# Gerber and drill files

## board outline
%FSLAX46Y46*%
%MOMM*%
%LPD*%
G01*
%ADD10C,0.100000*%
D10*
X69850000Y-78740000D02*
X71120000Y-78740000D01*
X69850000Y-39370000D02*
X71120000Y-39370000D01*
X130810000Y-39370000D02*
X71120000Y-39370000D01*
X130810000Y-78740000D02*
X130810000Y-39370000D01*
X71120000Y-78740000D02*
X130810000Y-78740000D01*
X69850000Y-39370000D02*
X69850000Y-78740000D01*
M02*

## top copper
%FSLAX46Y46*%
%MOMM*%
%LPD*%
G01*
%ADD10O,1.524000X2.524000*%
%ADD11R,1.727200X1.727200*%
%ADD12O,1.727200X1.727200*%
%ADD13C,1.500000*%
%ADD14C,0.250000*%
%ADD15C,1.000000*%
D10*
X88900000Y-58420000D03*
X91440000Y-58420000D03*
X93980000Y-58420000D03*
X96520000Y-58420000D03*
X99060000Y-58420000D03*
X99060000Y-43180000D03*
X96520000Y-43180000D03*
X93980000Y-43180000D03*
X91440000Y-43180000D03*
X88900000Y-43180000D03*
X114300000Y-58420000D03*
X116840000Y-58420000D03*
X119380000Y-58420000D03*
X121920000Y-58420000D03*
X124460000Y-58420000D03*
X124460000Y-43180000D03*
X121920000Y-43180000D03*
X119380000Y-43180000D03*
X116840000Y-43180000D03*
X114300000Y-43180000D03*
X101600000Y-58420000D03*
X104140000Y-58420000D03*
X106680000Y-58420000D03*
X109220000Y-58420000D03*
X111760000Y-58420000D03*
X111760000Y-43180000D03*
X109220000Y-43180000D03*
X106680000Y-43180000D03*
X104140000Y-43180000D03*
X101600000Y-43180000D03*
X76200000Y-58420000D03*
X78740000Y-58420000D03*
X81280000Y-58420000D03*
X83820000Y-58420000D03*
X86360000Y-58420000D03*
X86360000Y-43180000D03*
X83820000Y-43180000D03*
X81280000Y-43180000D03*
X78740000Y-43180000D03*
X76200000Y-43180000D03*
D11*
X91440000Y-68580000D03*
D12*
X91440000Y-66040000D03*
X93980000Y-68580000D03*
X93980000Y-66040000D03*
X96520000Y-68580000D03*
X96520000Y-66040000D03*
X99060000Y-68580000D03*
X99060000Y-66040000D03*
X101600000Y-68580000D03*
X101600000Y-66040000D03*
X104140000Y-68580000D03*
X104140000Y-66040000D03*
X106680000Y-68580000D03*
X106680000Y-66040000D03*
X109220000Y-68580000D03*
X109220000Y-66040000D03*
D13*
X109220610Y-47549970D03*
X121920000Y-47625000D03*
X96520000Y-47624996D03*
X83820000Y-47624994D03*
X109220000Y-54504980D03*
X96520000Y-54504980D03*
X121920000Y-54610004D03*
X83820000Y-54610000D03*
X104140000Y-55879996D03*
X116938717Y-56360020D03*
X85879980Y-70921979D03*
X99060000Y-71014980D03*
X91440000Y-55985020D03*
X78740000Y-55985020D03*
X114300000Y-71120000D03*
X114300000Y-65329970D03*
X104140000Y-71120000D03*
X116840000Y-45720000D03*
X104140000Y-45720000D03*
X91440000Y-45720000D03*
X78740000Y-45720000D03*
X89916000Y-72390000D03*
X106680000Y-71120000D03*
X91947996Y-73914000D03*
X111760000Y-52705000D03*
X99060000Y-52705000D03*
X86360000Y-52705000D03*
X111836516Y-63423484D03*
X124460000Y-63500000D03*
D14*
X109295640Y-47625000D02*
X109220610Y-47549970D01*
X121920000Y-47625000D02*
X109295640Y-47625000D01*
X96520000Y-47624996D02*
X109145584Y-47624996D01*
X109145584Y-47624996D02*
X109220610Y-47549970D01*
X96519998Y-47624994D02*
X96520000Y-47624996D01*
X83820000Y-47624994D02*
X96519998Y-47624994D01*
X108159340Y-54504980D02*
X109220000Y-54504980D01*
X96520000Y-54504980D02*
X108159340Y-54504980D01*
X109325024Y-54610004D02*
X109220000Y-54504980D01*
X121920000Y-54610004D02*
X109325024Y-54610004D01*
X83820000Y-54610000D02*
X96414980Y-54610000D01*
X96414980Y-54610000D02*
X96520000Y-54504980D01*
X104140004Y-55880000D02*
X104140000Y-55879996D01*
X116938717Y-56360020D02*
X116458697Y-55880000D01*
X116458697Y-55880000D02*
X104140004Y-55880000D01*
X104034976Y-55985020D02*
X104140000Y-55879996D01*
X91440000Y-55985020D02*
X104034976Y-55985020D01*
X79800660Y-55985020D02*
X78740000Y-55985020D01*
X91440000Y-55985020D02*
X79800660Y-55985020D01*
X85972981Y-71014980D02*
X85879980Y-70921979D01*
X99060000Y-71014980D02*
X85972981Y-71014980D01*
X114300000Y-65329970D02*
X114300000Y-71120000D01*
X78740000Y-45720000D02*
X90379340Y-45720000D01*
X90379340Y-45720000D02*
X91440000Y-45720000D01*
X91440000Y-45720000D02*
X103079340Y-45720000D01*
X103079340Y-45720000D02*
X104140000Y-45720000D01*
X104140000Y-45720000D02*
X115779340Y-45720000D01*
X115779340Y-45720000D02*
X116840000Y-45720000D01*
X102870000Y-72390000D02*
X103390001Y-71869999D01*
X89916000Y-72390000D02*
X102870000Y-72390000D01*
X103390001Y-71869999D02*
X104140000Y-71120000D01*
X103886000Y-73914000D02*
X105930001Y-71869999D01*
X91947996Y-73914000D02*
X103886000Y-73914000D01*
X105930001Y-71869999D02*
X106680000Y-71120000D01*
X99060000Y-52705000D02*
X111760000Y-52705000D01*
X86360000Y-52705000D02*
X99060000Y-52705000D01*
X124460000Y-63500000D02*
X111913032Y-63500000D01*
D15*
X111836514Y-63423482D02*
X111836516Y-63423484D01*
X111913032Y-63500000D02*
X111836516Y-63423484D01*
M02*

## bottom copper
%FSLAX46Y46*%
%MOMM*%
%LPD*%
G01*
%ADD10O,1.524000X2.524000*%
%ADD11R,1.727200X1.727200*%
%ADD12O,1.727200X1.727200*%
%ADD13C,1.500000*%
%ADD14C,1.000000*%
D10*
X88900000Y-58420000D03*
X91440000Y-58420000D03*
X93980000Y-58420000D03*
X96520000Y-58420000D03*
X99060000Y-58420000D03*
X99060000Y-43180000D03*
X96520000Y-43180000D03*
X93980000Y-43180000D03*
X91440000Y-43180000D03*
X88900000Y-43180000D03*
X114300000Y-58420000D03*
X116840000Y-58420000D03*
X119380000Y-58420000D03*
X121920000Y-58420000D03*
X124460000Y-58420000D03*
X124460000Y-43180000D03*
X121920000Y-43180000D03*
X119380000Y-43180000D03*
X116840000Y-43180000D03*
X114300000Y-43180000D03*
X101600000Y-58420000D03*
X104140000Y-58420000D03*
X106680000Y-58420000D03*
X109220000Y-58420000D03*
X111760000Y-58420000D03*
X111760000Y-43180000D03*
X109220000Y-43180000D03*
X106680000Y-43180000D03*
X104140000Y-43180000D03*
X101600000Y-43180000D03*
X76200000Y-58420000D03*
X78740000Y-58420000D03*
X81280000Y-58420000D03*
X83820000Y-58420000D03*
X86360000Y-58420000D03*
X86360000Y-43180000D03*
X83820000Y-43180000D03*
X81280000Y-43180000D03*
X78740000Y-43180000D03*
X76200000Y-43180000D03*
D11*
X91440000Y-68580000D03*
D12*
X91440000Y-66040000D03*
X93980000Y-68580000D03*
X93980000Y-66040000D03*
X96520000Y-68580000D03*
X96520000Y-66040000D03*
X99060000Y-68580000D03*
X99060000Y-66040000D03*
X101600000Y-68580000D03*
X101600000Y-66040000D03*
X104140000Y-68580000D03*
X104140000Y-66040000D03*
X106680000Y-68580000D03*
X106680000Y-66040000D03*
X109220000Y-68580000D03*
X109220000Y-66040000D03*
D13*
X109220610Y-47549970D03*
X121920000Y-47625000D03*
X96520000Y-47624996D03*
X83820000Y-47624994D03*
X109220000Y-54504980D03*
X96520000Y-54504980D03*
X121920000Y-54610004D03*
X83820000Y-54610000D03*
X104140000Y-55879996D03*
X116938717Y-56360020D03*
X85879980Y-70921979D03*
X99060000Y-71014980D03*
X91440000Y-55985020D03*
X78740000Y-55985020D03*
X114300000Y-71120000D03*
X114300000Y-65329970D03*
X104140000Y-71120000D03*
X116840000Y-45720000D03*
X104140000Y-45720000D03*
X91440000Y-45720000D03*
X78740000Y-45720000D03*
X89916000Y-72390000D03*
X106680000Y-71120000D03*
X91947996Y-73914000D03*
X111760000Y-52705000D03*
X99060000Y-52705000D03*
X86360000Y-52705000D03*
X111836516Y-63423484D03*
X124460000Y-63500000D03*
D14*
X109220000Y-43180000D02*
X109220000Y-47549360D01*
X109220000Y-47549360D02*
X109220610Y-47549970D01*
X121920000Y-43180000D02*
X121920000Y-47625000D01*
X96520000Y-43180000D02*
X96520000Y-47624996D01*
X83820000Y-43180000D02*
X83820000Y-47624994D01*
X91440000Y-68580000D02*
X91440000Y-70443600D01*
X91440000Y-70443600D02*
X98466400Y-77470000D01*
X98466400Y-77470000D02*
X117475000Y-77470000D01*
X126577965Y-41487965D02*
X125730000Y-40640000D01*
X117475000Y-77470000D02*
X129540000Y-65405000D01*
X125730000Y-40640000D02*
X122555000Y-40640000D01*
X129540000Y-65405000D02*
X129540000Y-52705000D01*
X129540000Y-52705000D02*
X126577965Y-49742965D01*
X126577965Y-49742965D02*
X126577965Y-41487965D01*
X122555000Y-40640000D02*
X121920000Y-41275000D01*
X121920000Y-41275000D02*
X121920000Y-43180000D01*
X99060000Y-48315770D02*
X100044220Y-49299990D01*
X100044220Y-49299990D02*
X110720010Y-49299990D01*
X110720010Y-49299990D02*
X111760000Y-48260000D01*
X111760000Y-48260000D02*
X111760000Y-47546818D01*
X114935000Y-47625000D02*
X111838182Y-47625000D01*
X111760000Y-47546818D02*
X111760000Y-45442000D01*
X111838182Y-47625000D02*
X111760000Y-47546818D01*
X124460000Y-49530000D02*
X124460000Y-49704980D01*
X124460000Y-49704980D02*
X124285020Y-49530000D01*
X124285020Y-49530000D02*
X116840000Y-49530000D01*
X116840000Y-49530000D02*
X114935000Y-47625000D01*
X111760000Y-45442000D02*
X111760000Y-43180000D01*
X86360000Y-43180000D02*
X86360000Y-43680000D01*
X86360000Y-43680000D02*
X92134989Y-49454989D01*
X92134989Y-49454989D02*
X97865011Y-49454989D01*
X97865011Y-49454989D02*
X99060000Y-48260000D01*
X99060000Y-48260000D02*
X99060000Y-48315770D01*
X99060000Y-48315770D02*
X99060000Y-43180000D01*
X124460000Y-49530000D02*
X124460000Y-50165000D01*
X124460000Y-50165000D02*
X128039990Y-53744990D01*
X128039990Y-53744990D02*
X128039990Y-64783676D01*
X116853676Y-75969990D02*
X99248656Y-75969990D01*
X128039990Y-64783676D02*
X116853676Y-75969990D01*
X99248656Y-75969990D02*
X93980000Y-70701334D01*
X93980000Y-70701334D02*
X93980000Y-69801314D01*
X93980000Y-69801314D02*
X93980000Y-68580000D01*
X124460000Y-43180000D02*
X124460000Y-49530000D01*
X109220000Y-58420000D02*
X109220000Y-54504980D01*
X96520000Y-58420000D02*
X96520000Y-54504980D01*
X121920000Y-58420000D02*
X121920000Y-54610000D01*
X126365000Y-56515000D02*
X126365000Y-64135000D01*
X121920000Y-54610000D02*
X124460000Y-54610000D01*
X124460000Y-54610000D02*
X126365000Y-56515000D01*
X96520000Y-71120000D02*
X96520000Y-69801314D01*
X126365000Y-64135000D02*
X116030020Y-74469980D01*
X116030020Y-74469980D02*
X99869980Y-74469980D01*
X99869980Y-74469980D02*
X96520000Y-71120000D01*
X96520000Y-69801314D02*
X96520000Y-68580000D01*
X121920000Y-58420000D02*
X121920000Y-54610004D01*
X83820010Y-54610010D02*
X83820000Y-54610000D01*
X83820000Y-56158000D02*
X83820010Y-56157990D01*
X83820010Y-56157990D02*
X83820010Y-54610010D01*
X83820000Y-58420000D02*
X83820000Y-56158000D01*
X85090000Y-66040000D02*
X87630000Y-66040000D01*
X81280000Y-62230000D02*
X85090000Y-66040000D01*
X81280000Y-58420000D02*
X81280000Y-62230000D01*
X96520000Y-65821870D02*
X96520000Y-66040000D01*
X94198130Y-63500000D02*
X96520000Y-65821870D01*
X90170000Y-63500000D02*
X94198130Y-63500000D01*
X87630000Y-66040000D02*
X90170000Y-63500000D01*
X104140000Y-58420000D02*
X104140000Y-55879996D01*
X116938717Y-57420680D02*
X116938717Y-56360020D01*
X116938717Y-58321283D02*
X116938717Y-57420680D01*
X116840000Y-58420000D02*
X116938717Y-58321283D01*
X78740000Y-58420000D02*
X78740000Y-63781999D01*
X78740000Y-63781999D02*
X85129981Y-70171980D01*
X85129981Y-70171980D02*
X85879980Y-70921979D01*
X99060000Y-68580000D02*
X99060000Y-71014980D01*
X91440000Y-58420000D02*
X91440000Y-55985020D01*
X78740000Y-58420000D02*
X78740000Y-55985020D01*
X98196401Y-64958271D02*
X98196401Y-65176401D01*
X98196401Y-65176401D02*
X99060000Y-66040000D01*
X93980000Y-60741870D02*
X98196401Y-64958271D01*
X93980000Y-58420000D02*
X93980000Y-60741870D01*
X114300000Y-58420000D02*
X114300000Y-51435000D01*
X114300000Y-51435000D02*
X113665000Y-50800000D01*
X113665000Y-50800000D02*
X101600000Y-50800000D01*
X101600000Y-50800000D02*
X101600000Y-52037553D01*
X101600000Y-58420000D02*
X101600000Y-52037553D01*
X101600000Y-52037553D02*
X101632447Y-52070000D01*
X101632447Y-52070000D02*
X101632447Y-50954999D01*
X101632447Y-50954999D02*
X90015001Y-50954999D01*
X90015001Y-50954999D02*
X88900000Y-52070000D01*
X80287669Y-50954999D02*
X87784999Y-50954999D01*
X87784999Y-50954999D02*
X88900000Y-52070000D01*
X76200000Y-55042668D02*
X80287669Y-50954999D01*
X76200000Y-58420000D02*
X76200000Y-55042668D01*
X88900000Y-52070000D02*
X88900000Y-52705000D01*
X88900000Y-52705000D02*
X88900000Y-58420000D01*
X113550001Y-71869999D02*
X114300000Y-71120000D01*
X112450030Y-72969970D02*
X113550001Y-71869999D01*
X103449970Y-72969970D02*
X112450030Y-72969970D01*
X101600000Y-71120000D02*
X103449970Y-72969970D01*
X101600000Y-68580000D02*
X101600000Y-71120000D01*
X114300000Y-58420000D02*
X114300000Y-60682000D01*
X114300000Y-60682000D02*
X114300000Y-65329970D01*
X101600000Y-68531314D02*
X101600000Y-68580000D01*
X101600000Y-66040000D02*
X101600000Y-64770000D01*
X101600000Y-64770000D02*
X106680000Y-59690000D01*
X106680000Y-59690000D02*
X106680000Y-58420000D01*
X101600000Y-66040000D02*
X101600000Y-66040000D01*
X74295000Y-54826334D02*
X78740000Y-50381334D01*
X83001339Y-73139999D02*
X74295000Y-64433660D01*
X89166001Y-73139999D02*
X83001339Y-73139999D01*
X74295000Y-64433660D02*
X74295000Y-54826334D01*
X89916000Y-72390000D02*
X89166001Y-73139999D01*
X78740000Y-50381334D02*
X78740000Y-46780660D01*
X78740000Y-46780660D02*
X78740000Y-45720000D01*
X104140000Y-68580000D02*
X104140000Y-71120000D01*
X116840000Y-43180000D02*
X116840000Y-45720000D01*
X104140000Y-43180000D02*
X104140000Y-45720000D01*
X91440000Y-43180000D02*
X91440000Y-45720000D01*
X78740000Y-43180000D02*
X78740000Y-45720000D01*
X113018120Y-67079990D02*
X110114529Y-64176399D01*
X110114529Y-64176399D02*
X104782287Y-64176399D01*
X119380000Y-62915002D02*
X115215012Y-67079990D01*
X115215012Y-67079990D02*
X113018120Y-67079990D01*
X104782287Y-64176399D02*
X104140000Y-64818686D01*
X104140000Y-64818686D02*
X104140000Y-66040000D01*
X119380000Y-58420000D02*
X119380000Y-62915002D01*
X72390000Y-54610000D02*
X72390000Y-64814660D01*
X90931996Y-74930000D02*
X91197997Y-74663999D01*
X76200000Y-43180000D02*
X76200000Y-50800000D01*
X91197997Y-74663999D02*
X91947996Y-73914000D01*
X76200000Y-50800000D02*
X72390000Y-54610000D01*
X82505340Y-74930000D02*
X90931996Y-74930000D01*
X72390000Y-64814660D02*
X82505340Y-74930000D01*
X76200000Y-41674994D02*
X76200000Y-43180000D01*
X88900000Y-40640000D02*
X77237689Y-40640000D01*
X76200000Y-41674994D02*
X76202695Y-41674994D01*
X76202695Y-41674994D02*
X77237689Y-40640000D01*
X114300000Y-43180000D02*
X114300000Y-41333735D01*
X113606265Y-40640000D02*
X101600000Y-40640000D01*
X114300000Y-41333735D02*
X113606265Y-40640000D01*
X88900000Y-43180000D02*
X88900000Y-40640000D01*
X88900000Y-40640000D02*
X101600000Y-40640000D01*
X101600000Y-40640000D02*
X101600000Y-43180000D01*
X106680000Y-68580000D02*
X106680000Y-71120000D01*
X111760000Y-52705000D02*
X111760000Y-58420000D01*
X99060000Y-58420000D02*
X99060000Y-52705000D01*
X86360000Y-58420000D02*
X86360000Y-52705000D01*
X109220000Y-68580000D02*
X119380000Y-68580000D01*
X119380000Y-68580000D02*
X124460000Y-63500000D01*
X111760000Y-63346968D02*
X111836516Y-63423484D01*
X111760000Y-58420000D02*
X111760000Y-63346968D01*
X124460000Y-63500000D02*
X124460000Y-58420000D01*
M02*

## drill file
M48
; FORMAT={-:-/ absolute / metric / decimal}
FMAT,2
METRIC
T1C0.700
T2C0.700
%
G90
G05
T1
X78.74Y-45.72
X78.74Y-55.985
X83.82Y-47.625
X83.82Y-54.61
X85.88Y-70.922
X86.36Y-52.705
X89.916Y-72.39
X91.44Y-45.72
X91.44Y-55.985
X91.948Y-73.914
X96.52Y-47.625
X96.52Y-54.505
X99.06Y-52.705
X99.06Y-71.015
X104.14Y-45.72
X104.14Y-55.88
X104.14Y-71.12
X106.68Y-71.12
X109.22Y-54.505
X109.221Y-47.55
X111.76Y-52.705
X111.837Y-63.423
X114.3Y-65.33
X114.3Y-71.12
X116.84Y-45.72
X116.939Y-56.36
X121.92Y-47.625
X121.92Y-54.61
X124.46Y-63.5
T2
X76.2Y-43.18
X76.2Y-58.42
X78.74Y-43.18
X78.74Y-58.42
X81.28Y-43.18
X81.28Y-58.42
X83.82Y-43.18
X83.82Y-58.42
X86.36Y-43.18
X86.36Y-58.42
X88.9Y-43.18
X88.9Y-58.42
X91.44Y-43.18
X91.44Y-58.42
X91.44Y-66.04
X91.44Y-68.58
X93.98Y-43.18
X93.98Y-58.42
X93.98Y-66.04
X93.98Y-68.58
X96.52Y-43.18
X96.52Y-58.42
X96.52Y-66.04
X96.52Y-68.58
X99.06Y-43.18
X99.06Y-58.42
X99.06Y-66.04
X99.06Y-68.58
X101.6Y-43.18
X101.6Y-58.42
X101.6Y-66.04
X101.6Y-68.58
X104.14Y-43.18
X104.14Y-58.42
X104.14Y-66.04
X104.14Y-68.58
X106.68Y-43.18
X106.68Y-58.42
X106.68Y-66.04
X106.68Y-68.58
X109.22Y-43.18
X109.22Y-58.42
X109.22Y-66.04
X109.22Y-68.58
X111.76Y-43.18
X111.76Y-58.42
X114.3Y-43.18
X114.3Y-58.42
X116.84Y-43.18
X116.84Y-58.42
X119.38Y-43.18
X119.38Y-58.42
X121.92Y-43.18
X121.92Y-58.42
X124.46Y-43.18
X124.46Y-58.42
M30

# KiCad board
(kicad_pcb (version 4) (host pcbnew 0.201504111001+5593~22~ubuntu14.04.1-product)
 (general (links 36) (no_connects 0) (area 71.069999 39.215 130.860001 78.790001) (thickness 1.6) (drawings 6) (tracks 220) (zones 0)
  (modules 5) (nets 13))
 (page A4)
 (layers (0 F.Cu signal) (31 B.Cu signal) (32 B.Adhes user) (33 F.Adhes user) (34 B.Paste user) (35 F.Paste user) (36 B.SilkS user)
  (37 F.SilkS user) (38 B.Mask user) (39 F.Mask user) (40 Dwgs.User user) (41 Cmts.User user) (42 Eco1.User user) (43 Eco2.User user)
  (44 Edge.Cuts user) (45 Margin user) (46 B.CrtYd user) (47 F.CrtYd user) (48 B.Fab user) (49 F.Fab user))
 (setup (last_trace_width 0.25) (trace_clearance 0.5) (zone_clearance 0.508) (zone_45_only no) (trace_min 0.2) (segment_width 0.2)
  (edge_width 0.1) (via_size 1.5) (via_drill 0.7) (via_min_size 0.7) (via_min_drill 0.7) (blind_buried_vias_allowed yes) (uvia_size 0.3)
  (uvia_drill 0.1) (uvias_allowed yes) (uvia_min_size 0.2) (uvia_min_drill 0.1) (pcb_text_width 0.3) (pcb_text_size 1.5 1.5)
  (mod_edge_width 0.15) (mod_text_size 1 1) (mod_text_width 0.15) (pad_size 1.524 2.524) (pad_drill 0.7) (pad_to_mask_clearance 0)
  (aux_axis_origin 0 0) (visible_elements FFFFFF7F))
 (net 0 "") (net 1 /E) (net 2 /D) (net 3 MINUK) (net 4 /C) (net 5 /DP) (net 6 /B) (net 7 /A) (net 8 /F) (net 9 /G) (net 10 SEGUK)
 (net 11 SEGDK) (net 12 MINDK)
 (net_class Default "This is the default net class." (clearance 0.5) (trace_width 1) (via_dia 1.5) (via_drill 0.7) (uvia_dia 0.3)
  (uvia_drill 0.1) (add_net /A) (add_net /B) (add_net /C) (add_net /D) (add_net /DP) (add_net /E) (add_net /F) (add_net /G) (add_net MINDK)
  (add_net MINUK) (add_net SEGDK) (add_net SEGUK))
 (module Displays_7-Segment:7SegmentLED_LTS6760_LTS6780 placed (layer F.Cu) (at 93.98 50.8)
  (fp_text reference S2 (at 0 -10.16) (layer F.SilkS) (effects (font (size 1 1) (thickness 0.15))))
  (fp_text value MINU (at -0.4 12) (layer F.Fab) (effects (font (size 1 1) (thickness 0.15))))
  (pad 1 thru_hole oval (at -5.08 7.62) (size 1.524 2.524) (drill 0.7) (layers *.Cu *.Mask F.SilkS) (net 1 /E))
  (pad 2 thru_hole oval (at -2.54 7.62) (size 1.524 2.524) (drill 0.7) (layers *.Cu *.Mask F.SilkS) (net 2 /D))
  (pad 3 thru_hole oval (at 0 7.62) (size 1.524 2.524) (drill 0.7) (layers *.Cu *.Mask F.SilkS) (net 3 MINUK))
  (pad 4 thru_hole oval (at 2.54 7.62) (size 1.524 2.524) (drill 0.7) (layers *.Cu *.Mask F.SilkS) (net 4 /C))
  (pad 5 thru_hole oval (at 5.08 7.62) (size 1.524 2.524) (drill 0.7) (layers *.Cu *.Mask F.SilkS) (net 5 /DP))
  (pad 6 thru_hole oval (at 5.08 -7.62) (size 1.524 2.524) (drill 0.7) (layers *.Cu *.Mask F.SilkS) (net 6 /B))
  (pad 7 thru_hole oval (at 2.54 -7.62) (size 1.524 2.524) (drill 0.7) (layers *.Cu *.Mask F.SilkS) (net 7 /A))
  (pad 8 thru_hole oval (at 0 -7.62) (size 1.524 2.524) (drill 0.7) (layers *.Cu *.Mask F.SilkS))
  (pad 9 thru_hole oval (at -2.54 -7.62) (size 1.524 2.524) (drill 0.7) (layers *.Cu *.Mask F.SilkS) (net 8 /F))
  (pad 10 thru_hole oval (at -5.08 -7.62) (size 1.524 2.524) (drill 0.7) (layers *.Cu *.Mask F.SilkS) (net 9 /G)))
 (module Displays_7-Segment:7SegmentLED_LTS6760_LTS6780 (layer F.Cu) (at 119.38 50.8)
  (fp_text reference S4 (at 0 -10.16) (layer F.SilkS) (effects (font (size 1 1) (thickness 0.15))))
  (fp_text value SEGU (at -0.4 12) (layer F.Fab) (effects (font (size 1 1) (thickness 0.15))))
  (pad 1 thru_hole oval (at -5.08 7.62) (size 1.524 2.524) (drill 0.7) (layers *.Cu *.Mask F.SilkS) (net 1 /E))
  (pad 2 thru_hole oval (at -2.54 7.62) (size 1.524 2.524) (drill 0.7) (layers *.Cu *.Mask F.SilkS) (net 2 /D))
  (pad 3 thru_hole oval (at 0 7.62) (size 1.524 2.524) (drill 0.7) (layers *.Cu *.Mask F.SilkS) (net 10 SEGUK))
  (pad 4 thru_hole oval (at 2.54 7.62) (size 1.524 2.524) (drill 0.7) (layers *.Cu *.Mask F.SilkS) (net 4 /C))
  (pad 5 thru_hole oval (at 5.08 7.62) (size 1.524 2.524) (drill 0.7) (layers *.Cu *.Mask F.SilkS) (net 5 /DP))
  (pad 6 thru_hole oval (at 5.08 -7.62) (size 1.524 2.524) (drill 0.7) (layers *.Cu *.Mask F.SilkS) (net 6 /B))
  (pad 7 thru_hole oval (at 2.54 -7.62) (size 1.524 2.524) (drill 0.7) (layers *.Cu *.Mask F.SilkS) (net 7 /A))
  (pad 8 thru_hole oval (at 0 -7.62) (size 1.524 2.524) (drill 0.7) (layers *.Cu *.Mask F.SilkS))
  (pad 9 thru_hole oval (at -2.54 -7.62) (size 1.524 2.524) (drill 0.7) (layers *.Cu *.Mask F.SilkS) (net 8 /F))
  (pad 10 thru_hole oval (at -5.08 -7.62) (size 1.524 2.524) (drill 0.7) (layers *.Cu *.Mask F.SilkS) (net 9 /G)))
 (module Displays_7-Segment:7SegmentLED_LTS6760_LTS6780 (layer F.Cu) (at 106.68 50.8)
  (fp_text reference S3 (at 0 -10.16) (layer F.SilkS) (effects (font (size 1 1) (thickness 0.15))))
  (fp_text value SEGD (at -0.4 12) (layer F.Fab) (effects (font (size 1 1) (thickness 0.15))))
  (pad 1 thru_hole oval (at -5.08 7.62) (size 1.524 2.524) (drill 0.7) (layers *.Cu *.Mask F.SilkS) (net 1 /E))
  (pad 2 thru_hole oval (at -2.54 7.62) (size 1.524 2.524) (drill 0.7) (layers *.Cu *.Mask F.SilkS) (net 2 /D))
  (pad 3 thru_hole oval (at 0 7.62) (size 1.524 2.524) (drill 0.7) (layers *.Cu *.Mask F.SilkS) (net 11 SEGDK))
  (pad 4 thru_hole oval (at 2.54 7.62) (size 1.524 2.524) (drill 0.7) (layers *.Cu *.Mask F.SilkS) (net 4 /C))
  (pad 5 thru_hole oval (at 5.08 7.62) (size 1.524 2.524) (drill 0.7) (layers *.Cu *.Mask F.SilkS) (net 5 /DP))
  (pad 6 thru_hole oval (at 5.08 -7.62) (size 1.524 2.524) (drill 0.7) (layers *.Cu *.Mask F.SilkS) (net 6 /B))
  (pad 7 thru_hole oval (at 2.54 -7.62) (size 1.524 2.524) (drill 0.7) (layers *.Cu *.Mask F.SilkS) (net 7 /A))
  (pad 8 thru_hole oval (at 0 -7.62) (size 1.524 2.524) (drill 0.7) (layers *.Cu *.Mask F.SilkS))
  (pad 9 thru_hole oval (at -2.54 -7.62) (size 1.524 2.524) (drill 0.7) (layers *.Cu *.Mask F.SilkS) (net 8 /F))
  (pad 10 thru_hole oval (at -5.08 -7.62) (size 1.524 2.524) (drill 0.7) (layers *.Cu *.Mask F.SilkS) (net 9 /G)))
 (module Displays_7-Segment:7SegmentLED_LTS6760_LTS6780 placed (layer F.Cu) (at 81.28 50.8)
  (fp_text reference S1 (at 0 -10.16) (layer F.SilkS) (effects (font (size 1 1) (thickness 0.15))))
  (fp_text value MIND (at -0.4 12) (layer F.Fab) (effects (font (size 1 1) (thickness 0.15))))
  (pad 1 thru_hole oval (at -5.08 7.62) (size 1.524 2.524) (drill 0.7) (layers *.Cu *.Mask F.SilkS) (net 1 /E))
  (pad 2 thru_hole oval (at -2.54 7.62) (size 1.524 2.524) (drill 0.7) (layers *.Cu *.Mask F.SilkS) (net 2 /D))
  (pad 3 thru_hole oval (at 0 7.62) (size 1.524 2.524) (drill 0.7) (layers *.Cu *.Mask F.SilkS) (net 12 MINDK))
  (pad 4 thru_hole oval (at 2.54 7.62) (size 1.524 2.524) (drill 0.7) (layers *.Cu *.Mask F.SilkS) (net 4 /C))
  (pad 5 thru_hole oval (at 5.08 7.62) (size 1.524 2.524) (drill 0.7) (layers *.Cu *.Mask F.SilkS) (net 5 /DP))
  (pad 6 thru_hole oval (at 5.08 -7.62) (size 1.524 2.524) (drill 0.7) (layers *.Cu *.Mask F.SilkS) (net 6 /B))
  (pad 7 thru_hole oval (at 2.54 -7.62) (size 1.524 2.524) (drill 0.7) (layers *.Cu *.Mask F.SilkS) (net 7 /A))
  (pad 8 thru_hole oval (at 0 -7.62) (size 1.524 2.524) (drill 0.7) (layers *.Cu *.Mask F.SilkS))
  (pad 9 thru_hole oval (at -2.54 -7.62) (size 1.524 2.524) (drill 0.7) (layers *.Cu *.Mask F.SilkS) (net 8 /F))
  (pad 10 thru_hole oval (at -5.08 -7.62) (size 1.524 2.524) (drill 0.7) (layers *.Cu *.Mask F.SilkS) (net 9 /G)))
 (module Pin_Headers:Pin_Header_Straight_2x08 (layer F.Cu) (at 91.44 68.58 90)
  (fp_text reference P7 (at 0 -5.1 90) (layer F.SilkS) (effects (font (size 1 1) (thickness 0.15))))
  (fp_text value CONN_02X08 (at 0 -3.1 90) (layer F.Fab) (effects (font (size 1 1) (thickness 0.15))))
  (pad 1 thru_hole rect (at 0 0 90) (size 1.7272 1.7272) (drill 0.7) (layers *.Cu *.Mask F.SilkS) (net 7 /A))
  (pad 2 thru_hole oval (at 2.54 0 90) (size 1.7272 1.7272) (drill 0.7) (layers *.Cu *.Mask F.SilkS))
  (pad 3 thru_hole oval (at 0 2.54 90) (size 1.7272 1.7272) (drill 0.7) (layers *.Cu *.Mask F.SilkS) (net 6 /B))
  (pad 4 thru_hole oval (at 2.54 2.54 90) (size 1.7272 1.7272) (drill 0.7) (layers *.Cu *.Mask F.SilkS))
  (pad 5 thru_hole oval (at 0 5.08 90) (size 1.7272 1.7272) (drill 0.7) (layers *.Cu *.Mask F.SilkS) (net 4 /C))
  (pad 6 thru_hole oval (at 2.54 5.08 90) (size 1.7272 1.7272) (drill 0.7) (layers *.Cu *.Mask F.SilkS) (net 12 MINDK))
  (pad 7 thru_hole oval (at 0 7.62 90) (size 1.7272 1.7272) (drill 0.7) (layers *.Cu *.Mask F.SilkS) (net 2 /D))
  (pad 8 thru_hole oval (at 2.54 7.62 90) (size 1.7272 1.7272) (drill 0.7) (layers *.Cu *.Mask F.SilkS) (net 3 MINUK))
  (pad 9 thru_hole oval (at 0 10.16 90) (size 1.7272 1.7272) (drill 0.7) (layers *.Cu *.Mask F.SilkS) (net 1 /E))
  (pad 10 thru_hole oval (at 2.54 10.16 90) (size 1.7272 1.7272) (drill 0.7) (layers *.Cu *.Mask F.SilkS) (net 11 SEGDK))
  (pad 11 thru_hole oval (at 0 12.7 90) (size 1.7272 1.7272) (drill 0.7) (layers *.Cu *.Mask F.SilkS) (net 8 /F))
  (pad 12 thru_hole oval (at 2.54 12.7 90) (size 1.7272 1.7272) (drill 0.7) (layers *.Cu *.Mask F.SilkS) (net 10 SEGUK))
  (pad 13 thru_hole oval (at 0 15.24 90) (size 1.7272 1.7272) (drill 0.7) (layers *.Cu *.Mask F.SilkS) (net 9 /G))
  (pad 14 thru_hole oval (at 2.54 15.24 90) (size 1.7272 1.7272) (drill 0.7) (layers *.Cu *.Mask F.SilkS))
  (pad 15 thru_hole oval (at 0 17.78 90) (size 1.7272 1.7272) (drill 0.7) (layers *.Cu *.Mask F.SilkS) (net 5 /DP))
  (pad 16 thru_hole oval (at 2.54 17.78 90) (size 1.7272 1.7272) (drill 0.7) (layers *.Cu *.Mask F.SilkS)))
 (gr_line (start 69.85 78.74) (end 71.12 78.74) (layer Edge.Cuts) (width 0.1))
 (gr_line (start 69.85 39.37) (end 71.12 39.37) (layer Edge.Cuts) (width 0.1))
 (gr_line (start 130.81 39.37) (end 71.12 39.37) (layer Edge.Cuts) (width 0.1))
 (gr_line (start 130.81 78.74) (end 130.81 39.37) (layer Edge.Cuts) (width 0.1))
 (gr_line (start 71.12 78.74) (end 130.81 78.74) (layer Edge.Cuts) (width 0.1))
 (gr_line (start 69.85 39.37) (end 69.85 78.74) (layer Edge.Cuts) (width 0.1))
 (via (at 109.22061 47.54997) (size 1.5) (drill 0.7) (layers F.Cu B.Cu) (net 7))
 (segment (start 109.22 43.18) (end 109.22 47.54936) (width 1) (layer B.Cu) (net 7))
 (segment (start 109.22 47.54936) (end 109.22061 47.54997) (width 1) (layer B.Cu) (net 7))
 (segment (start 109.29564 47.625) (end 109.22061 47.54997) (width 0.25) (layer F.Cu) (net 7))
 (segment (start 121.92 47.625) (end 109.29564 47.625) (width 0.25) (layer F.Cu) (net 7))
 (segment (start 96.52 47.624996) (end 109.145584 47.624996) (width 0.25) (layer F.Cu) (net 7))
 (segment (start 109.145584 47.624996) (end 109.22061 47.54997) (width 0.25) (layer F.Cu) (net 7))
 (segment (start 121.92 43.18) (end 121.92 47.625) (width 1) (layer B.Cu) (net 7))
 (via (at 121.92 47.625) (size 1.5) (drill 0.7) (layers F.Cu B.Cu) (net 7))
 (segment (start 96.519998 47.624994) (end 96.52 47.624996) (width 0.25) (layer F.Cu) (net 7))
 (segment (start 83.82 47.624994) (end 96.519998 47.624994) (width 0.25) (layer F.Cu) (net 7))
 (via (at 96.52 47.624996) (size 1.5) (drill 0.7) (layers F.Cu B.Cu) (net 7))
 (segment (start 96.52 43.18) (end 96.52 47.624996) (width 1) (layer B.Cu) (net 7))
 (segment (start 83.82 43.18) (end 83.82 47.624994) (width 1) (layer B.Cu) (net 7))
 (via (at 83.82 47.624994) (size 1.5) (drill 0.7) (layers F.Cu B.Cu) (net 7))
 (segment (start 91.44 68.58) (end 91.44 70.4436) (width 1) (layer B.Cu) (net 7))
 (segment (start 91.44 70.4436) (end 98.4664 77.47) (width 1) (layer B.Cu) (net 7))
 (segment (start 98.4664 77.47) (end 117.475 77.47) (width 1) (layer B.Cu) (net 7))
 (segment (start 126.577965 41.487965) (end 125.73 40.64) (width 1) (layer B.Cu) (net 7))
 (segment (start 117.475 77.47) (end 129.54 65.405) (width 1) (layer B.Cu) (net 7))
 (segment (start 125.73 40.64) (end 122.555 40.64) (width 1) (layer B.Cu) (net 7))
 (segment (start 129.54 65.405) (end 129.54 52.705) (width 1) (layer B.Cu) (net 7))
 (segment (start 129.54 52.705) (end 126.577965 49.742965) (width 1) (layer B.Cu) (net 7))
 (segment (start 126.577965 49.742965) (end 126.577965 41.487965) (width 1) (layer B.Cu) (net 7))
 (segment (start 122.555 40.64) (end 121.92 41.275) (width 1) (layer B.Cu) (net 7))
 (segment (start 121.92 41.275) (end 121.92 43.18) (width 1) (layer B.Cu) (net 7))
 (segment (start 99.06 48.31577) (end 100.04422 49.29999) (width 1) (layer B.Cu) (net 6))
 (segment (start 100.04422 49.29999) (end 110.72001 49.29999) (width 1) (layer B.Cu) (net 6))
 (segment (start 110.72001 49.29999) (end 111.76 48.26) (width 1) (layer B.Cu) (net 6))
 (segment (start 111.76 48.26) (end 111.76 47.546818) (width 1) (layer B.Cu) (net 6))
 (segment (start 114.935 47.625) (end 111.838182 47.625) (width 1) (layer B.Cu) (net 6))
 (segment (start 111.76 47.546818) (end 111.76 45.442) (width 1) (layer B.Cu) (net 6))
 (segment (start 111.838182 47.625) (end 111.76 47.546818) (width 1) (layer B.Cu) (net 6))
 (segment (start 124.46 49.53) (end 124.46 49.70498) (width 1) (layer B.Cu) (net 6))
 (segment (start 124.46 49.70498) (end 124.28502 49.53) (width 1) (layer B.Cu) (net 6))
 (segment (start 124.28502 49.53) (end 116.84 49.53) (width 1) (layer B.Cu) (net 6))
 (segment (start 116.84 49.53) (end 114.935 47.625) (width 1) (layer B.Cu) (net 6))
 (segment (start 111.76 45.442) (end 111.76 43.18) (width 1) (layer B.Cu) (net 6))
 (segment (start 86.36 43.18) (end 86.36 43.68) (width 1) (layer B.Cu) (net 6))
 (segment (start 86.36 43.68) (end 92.134989 49.454989) (width 1) (layer B.Cu) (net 6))
 (segment (start 92.134989 49.454989) (end 97.865011 49.454989) (width 1) (layer B.Cu) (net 6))
 (segment (start 97.865011 49.454989) (end 99.06 48.26) (width 1) (layer B.Cu) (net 6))
 (segment (start 99.06 48.26) (end 99.06 48.31577) (width 1) (layer B.Cu) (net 6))
 (segment (start 99.06 48.31577) (end 99.06 43.18) (width 1) (layer B.Cu) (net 6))
 (segment (start 124.46 49.53) (end 124.46 50.165) (width 1) (layer B.Cu) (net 6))
 (segment (start 124.46 50.165) (end 128.03999 53.74499) (width 1) (layer B.Cu) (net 6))
 (segment (start 128.03999 53.74499) (end 128.03999 64.783676) (width 1) (layer B.Cu) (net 6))
 (segment (start 116.853676 75.96999) (end 99.248656 75.96999) (width 1) (layer B.Cu) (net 6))
 (segment (start 128.03999 64.783676) (end 116.853676 75.96999) (width 1) (layer B.Cu) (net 6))
 (segment (start 99.248656 75.96999) (end 93.98 70.701334) (width 1) (layer B.Cu) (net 6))
 (segment (start 93.98 70.701334) (end 93.98 69.801314) (width 1) (layer B.Cu) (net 6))
 (segment (start 93.98 69.801314) (end 93.98 68.58) (width 1) (layer B.Cu) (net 6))
 (segment (start 124.46 43.18) (end 124.46 49.53) (width 1) (layer B.Cu) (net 6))
 (segment (start 108.15934 54.50498) (end 109.22 54.50498) (width 0.25) (layer F.Cu) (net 4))
 (segment (start 96.52 54.50498) (end 108.15934 54.50498) (width 0.25) (layer F.Cu) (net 4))
 (segment (start 109.325024 54.610004) (end 109.22 54.50498) (width 0.25) (layer F.Cu) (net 4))
 (segment (start 121.92 54.610004) (end 109.325024 54.610004) (width 0.25) (layer F.Cu) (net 4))
 (segment (start 109.22 58.42) (end 109.22 54.50498) (width 1) (layer B.Cu) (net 4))
 (via (at 109.22 54.50498) (size 1.5) (drill 0.7) (layers F.Cu B.Cu) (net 4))
 (segment (start 83.82 54.61) (end 96.41498 54.61) (width 0.25) (layer F.Cu) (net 4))
 (via (at 96.52 54.50498) (size 1.5) (drill 0.7) (layers F.Cu B.Cu) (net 4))
 (segment (start 96.41498 54.61) (end 96.52 54.50498) (width 0.25) (layer F.Cu) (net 4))
 (segment (start 96.52 58.42) (end 96.52 54.50498) (width 1) (layer B.Cu) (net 4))
 (segment (start 121.92 58.42) (end 121.92 54.61) (width 1) (layer B.Cu) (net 4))
 (segment (start 126.365 56.515) (end 126.365 64.135) (width 1) (layer B.Cu) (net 4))
 (segment (start 121.92 54.61) (end 124.46 54.61) (width 1) (layer B.Cu) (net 4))
 (segment (start 124.46 54.61) (end 126.365 56.515) (width 1) (layer B.Cu) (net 4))
 (segment (start 96.52 71.12) (end 96.52 69.801314) (width 1) (layer B.Cu) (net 4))
 (segment (start 126.365 64.135) (end 116.03002 74.46998) (width 1) (layer B.Cu) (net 4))
 (segment (start 116.03002 74.46998) (end 99.86998 74.46998) (width 1) (layer B.Cu) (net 4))
 (segment (start 99.86998 74.46998) (end 96.52 71.12) (width 1) (layer B.Cu) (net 4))
 (segment (start 96.52 69.801314) (end 96.52 68.58) (width 1) (layer B.Cu) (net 4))
 (segment (start 121.92 58.42) (end 121.92 54.610004) (width 1) (layer B.Cu) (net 4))
 (via (at 121.92 54.610004) (size 1.5) (drill 0.7) (layers F.Cu B.Cu) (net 4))
 (segment (start 83.82001 54.61001) (end 83.82 54.61) (width 1) (layer B.Cu) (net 4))
 (segment (start 83.82 56.158) (end 83.82001 56.15799) (width 1) (layer B.Cu) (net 4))
 (segment (start 83.82001 56.15799) (end 83.82001 54.61001) (width 1) (layer B.Cu) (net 4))
 (via (at 83.82 54.61) (size 1.5) (drill 0.7) (layers F.Cu B.Cu) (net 4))
 (segment (start 83.82 58.42) (end 83.82 56.158) (width 1) (layer B.Cu) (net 4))
 (segment (start 85.09 66.04) (end 87.63 66.04) (width 1) (layer B.Cu) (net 12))
 (segment (start 81.28 62.23) (end 85.09 66.04) (width 1) (layer B.Cu) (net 12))
 (segment (start 81.28 58.42) (end 81.28 62.23) (width 1) (layer B.Cu) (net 12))
 (segment (start 96.52 65.82187) (end 96.52 66.04) (width 1) (layer B.Cu) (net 12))
 (segment (start 94.19813 63.5) (end 96.52 65.82187) (width 1) (layer B.Cu) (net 12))
 (segment (start 90.17 63.5) (end 94.19813 63.5) (width 1) (layer B.Cu) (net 12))
 (segment (start 87.63 66.04) (end 90.17 63.5) (width 1) (layer B.Cu) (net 12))
 (segment (start 104.140004 55.88) (end 104.14 55.879996) (width 0.25) (layer F.Cu) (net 2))
 (segment (start 116.938717 56.36002) (end 116.458697 55.88) (width 0.25) (layer F.Cu) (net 2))
 (segment (start 116.458697 55.88) (end 104.140004 55.88) (width 0.25) (layer F.Cu) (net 2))
 (segment (start 104.034976 55.98502) (end 104.14 55.879996) (width 0.25) (layer F.Cu) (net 2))
 (segment (start 91.44 55.98502) (end 104.034976 55.98502) (width 0.25) (layer F.Cu) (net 2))
 (segment (start 104.14 58.42) (end 104.14 55.879996) (width 1) (layer B.Cu) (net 2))
 (via (at 104.14 55.879996) (size 1.5) (drill 0.7) (layers F.Cu B.Cu) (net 2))
 (segment (start 116.938717 57.42068) (end 116.938717 56.36002) (width 1) (layer B.Cu) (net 2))
 (segment (start 116.938717 58.321283) (end 116.938717 57.42068) (width 1) (layer B.Cu) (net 2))
 (segment (start 116.84 58.42) (end 116.938717 58.321283) (width 1) (layer B.Cu) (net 2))
 (via (at 116.938717 56.36002) (size 1.5) (drill 0.7) (layers F.Cu B.Cu) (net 2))
 (segment (start 79.80066 55.98502) (end 78.74 55.98502) (width 0.25) (layer F.Cu) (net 2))
 (segment (start 91.44 55.98502) (end 79.80066 55.98502) (width 0.25) (layer F.Cu) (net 2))
 (segment (start 85.972981 71.01498) (end 85.87998 70.921979) (width 0.25) (layer F.Cu) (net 2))
 (via (at 85.87998 70.921979) (size 1.5) (drill 0.7) (layers F.Cu B.Cu) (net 2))
 (segment (start 78.74 58.42) (end 78.74 63.781999) (width 1) (layer B.Cu) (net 2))
 (segment (start 78.74 63.781999) (end 85.129981 70.17198) (width 1) (layer B.Cu) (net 2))
 (segment (start 85.129981 70.17198) (end 85.87998 70.921979) (width 1) (layer B.Cu) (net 2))
 (segment (start 99.06 71.01498) (end 85.972981 71.01498) (width 0.25) (layer F.Cu) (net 2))
 (via (at 99.06 71.01498) (size 1.5) (drill 0.7) (layers F.Cu B.Cu) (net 2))
 (segment (start 99.06 68.58) (end 99.06 71.01498) (width 1) (layer B.Cu) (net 2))
 (segment (start 91.44 58.42) (end 91.44 55.98502) (width 1) (layer B.Cu) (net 2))
 (via (at 91.44 55.98502) (size 1.5) (drill 0.7) (layers F.Cu B.Cu) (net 2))
 (segment (start 78.74 58.42) (end 78.74 55.98502) (width 1) (layer B.Cu) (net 2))
 (via (at 78.74 55.98502) (size 1.5) (drill 0.7) (layers F.Cu B.Cu) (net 2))
 (segment (start 98.196401 64.958271) (end 98.196401 65.176401) (width 1) (layer B.Cu) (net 3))
 (segment (start 98.196401 65.176401) (end 99.06 66.04) (width 1) (layer B.Cu) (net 3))
 (segment (start 93.98 60.74187) (end 98.196401 64.958271) (width 1) (layer B.Cu) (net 3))
 (segment (start 93.98 58.42) (end 93.98 60.74187) (width 1) (layer B.Cu) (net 3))
 (segment (start 114.3 58.42) (end 114.3 51.435) (width 1) (layer B.Cu) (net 1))
 (segment (start 114.3 51.435) (end 113.665 50.8) (width 1) (layer B.Cu) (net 1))
 (segment (start 113.665 50.8) (end 101.6 50.8) (width 1) (layer B.Cu) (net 1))
 (segment (start 101.6 50.8) (end 101.6 52.037553) (width 1) (layer B.Cu) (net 1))
 (segment (start 101.6 58.42) (end 101.6 52.037553) (width 1) (layer B.Cu) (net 1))
 (segment (start 101.6 52.037553) (end 101.632447 52.07) (width 1) (layer B.Cu) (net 1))
 (segment (start 101.632447 52.07) (end 101.632447 50.954999) (width 1) (layer B.Cu) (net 1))
 (segment (start 101.632447 50.954999) (end 90.015001 50.954999) (width 1) (layer B.Cu) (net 1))
 (segment (start 90.015001 50.954999) (end 88.9 52.07) (width 1) (layer B.Cu) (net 1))
 (segment (start 80.287669 50.954999) (end 87.784999 50.954999) (width 1) (layer B.Cu) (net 1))
 (segment (start 87.784999 50.954999) (end 88.9 52.07) (width 1) (layer B.Cu) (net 1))
 (segment (start 76.2 55.042668) (end 80.287669 50.954999) (width 1) (layer B.Cu) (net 1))
 (segment (start 76.2 58.42) (end 76.2 55.042668) (width 1) (layer B.Cu) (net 1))
 (segment (start 88.9 52.07) (end 88.9 52.705) (width 1) (layer B.Cu) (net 1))
 (segment (start 88.9 52.705) (end 88.9 58.42) (width 1) (layer B.Cu) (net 1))
 (segment (start 113.550001 71.869999) (end 114.3 71.12) (width 1) (layer B.Cu) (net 1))
 (segment (start 112.45003 72.96997) (end 113.550001 71.869999) (width 1) (layer B.Cu) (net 1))
 (segment (start 103.44997 72.96997) (end 112.45003 72.96997) (width 1) (layer B.Cu) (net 1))
 (segment (start 101.6 71.12) (end 103.44997 72.96997) (width 1) (layer B.Cu) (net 1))
 (segment (start 101.6 68.58) (end 101.6 71.12) (width 1) (layer B.Cu) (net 1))
 (segment (start 114.3 65.32997) (end 114.3 71.12) (width 0.25) (layer F.Cu) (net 1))
 (via (at 114.3 71.12) (size 1.5) (drill 0.7) (layers F.Cu B.Cu) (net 1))
 (segment (start 114.3 58.42) (end 114.3 60.682) (width 1) (layer B.Cu) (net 1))
 (via (at 114.3 65.32997) (size 1.5) (drill 0.7) (layers F.Cu B.Cu) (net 1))
 (segment (start 114.3 60.682) (end 114.3 65.32997) (width 1) (layer B.Cu) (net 1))
 (segment (start 101.6 68.531314) (end 101.6 68.58) (width 1) (layer B.Cu) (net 1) (status 30))
 (segment (start 101.6 66.04) (end 101.6 64.77) (width 1) (layer B.Cu) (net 11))
 (segment (start 101.6 64.77) (end 106.68 59.69) (width 1) (layer B.Cu) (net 11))
 (segment (start 106.68 59.69) (end 106.68 58.42) (width 1) (layer B.Cu) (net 11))
 (segment (start 101.6 66.04) (end 101.6 66.04) (width 1) (layer B.Cu) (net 11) (status 20))
 (segment (start 78.74 45.72) (end 90.37934 45.72) (width 0.25) (layer F.Cu) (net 8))
 (segment (start 90.37934 45.72) (end 91.44 45.72) (width 0.25) (layer F.Cu) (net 8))
 (segment (start 91.44 45.72) (end 103.07934 45.72) (width 0.25) (layer F.Cu) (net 8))
 (segment (start 103.07934 45.72) (end 104.14 45.72) (width 0.25) (layer F.Cu) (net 8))
 (segment (start 104.14 45.72) (end 115.77934 45.72) (width 0.25) (layer F.Cu) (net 8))
 (segment (start 115.77934 45.72) (end 116.84 45.72) (width 0.25) (layer F.Cu) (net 8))
 (segment (start 74.295 54.826334) (end 78.74 50.381334) (width 1) (layer B.Cu) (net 8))
 (segment (start 83.001339 73.139999) (end 74.295 64.43366) (width 1) (layer B.Cu) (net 8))
 (segment (start 89.166001 73.139999) (end 83.001339 73.139999) (width 1) (layer B.Cu) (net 8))
 (segment (start 74.295 64.43366) (end 74.295 54.826334) (width 1) (layer B.Cu) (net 8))
 (segment (start 89.916 72.39) (end 89.166001 73.139999) (width 1) (layer B.Cu) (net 8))
 (segment (start 78.74 50.381334) (end 78.74 46.78066) (width 1) (layer B.Cu) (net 8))
 (segment (start 78.74 46.78066) (end 78.74 45.72) (width 1) (layer B.Cu) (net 8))
 (segment (start 102.87 72.39) (end 103.390001 71.869999) (width 0.25) (layer F.Cu) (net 8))
 (segment (start 89.916 72.39) (end 102.87 72.39) (width 0.25) (layer F.Cu) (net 8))
 (segment (start 104.14 68.58) (end 104.14 71.12) (width 1) (layer B.Cu) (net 8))
 (segment (start 103.390001 71.869999) (end 104.14 71.12) (width 0.25) (layer F.Cu) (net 8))
 (via (at 104.14 71.12) (size 1.5) (drill 0.7) (layers F.Cu B.Cu) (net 8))
 (segment (start 116.84 43.18) (end 116.84 45.72) (width 1) (layer B.Cu) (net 8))
 (via (at 116.84 45.72) (size 1.5) (drill 0.7) (layers F.Cu B.Cu) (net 8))
 (segment (start 104.14 43.18) (end 104.14 45.72) (width 1) (layer B.Cu) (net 8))
 (via (at 104.14 45.72) (size 1.5) (drill 0.7) (layers F.Cu B.Cu) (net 8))
 (segment (start 91.44 43.18) (end 91.44 45.72) (width 1) (layer B.Cu) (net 8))
 (via (at 91.44 45.72) (size 1.5) (drill 0.7) (layers F.Cu B.Cu) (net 8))
 (segment (start 78.74 43.18) (end 78.74 45.72) (width 1) (layer B.Cu) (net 8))
 (via (at 78.74 45.72) (size 1.5) (drill 0.7) (layers F.Cu B.Cu) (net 8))
 (via (at 89.916 72.39) (size 1.5) (drill 0.7) (layers F.Cu B.Cu) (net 8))
 (segment (start 113.01812 67.07999) (end 110.114529 64.176399) (width 1) (layer B.Cu) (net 10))
 (segment (start 110.114529 64.176399) (end 104.782287 64.176399) (width 1) (layer B.Cu) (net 10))
 (segment (start 119.38 62.915002) (end 115.215012 67.07999) (width 1) (layer B.Cu) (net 10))
 (segment (start 115.215012 67.07999) (end 113.01812 67.07999) (width 1) (layer B.Cu) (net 10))
 (segment (start 104.782287 64.176399) (end 104.14 64.818686) (width 1) (layer B.Cu) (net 10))
 (segment (start 104.14 64.818686) (end 104.14 66.04) (width 1) (layer B.Cu) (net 10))
 (segment (start 119.38 58.42) (end 119.38 62.915002) (width 1) (layer B.Cu) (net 10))
 (segment (start 72.39 54.61) (end 72.39 64.81466) (width 1) (layer B.Cu) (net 9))
 (segment (start 90.931996 74.93) (end 91.197997 74.663999) (width 1) (layer B.Cu) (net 9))
 (segment (start 76.2 43.18) (end 76.2 50.8) (width 1) (layer B.Cu) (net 9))
 (segment (start 91.197997 74.663999) (end 91.947996 73.914) (width 1) (layer B.Cu) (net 9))
 (segment (start 76.2 50.8) (end 72.39 54.61) (width 1) (layer B.Cu) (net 9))
 (segment (start 82.50534 74.93) (end 90.931996 74.93) (width 1) (layer B.Cu) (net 9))
 (segment (start 72.39 64.81466) (end 82.50534 74.93) (width 1) (layer B.Cu) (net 9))
 (segment (start 76.2 41.674994) (end 76.2 43.18) (width 1) (layer B.Cu) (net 9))
 (segment (start 88.9 40.64) (end 77.237689 40.64) (width 1) (layer B.Cu) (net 9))
 (segment (start 76.2 41.674994) (end 76.202695 41.674994) (width 1) (layer B.Cu) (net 9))
 (segment (start 76.202695 41.674994) (end 77.237689 40.64) (width 1) (layer B.Cu) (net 9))
 (segment (start 114.3 43.18) (end 114.3 41.333735) (width 1) (layer B.Cu) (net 9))
 (segment (start 113.606265 40.64) (end 101.6 40.64) (width 1) (layer B.Cu) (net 9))
 (segment (start 114.3 41.333735) (end 113.606265 40.64) (width 1) (layer B.Cu) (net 9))
 (segment (start 88.9 43.18) (end 88.9 40.64) (width 1) (layer B.Cu) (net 9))
 (segment (start 88.9 40.64) (end 101.6 40.64) (width 1) (layer B.Cu) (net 9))
 (segment (start 101.6 40.64) (end 101.6 43.18) (width 1) (layer B.Cu) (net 9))
 (segment (start 103.886 73.914) (end 105.930001 71.869999) (width 0.25) (layer F.Cu) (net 9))
 (segment (start 91.947996 73.914) (end 103.886 73.914) (width 0.25) (layer F.Cu) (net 9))
 (segment (start 105.930001 71.869999) (end 106.68 71.12) (width 0.25) (layer F.Cu) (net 9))
 (segment (start 106.68 68.58) (end 106.68 71.12) (width 1) (layer B.Cu) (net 9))
 (via (at 106.68 71.12) (size 1.5) (drill 0.7) (layers F.Cu B.Cu) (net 9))
 (via (at 91.947996 73.914) (size 1.5) (drill 0.7) (layers F.Cu B.Cu) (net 9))
 (segment (start 111.76 52.705) (end 111.76 58.42) (width 1) (layer B.Cu) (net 5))
 (segment (start 99.06 52.705) (end 111.76 52.705) (width 0.25) (layer F.Cu) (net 5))
 (via (at 111.76 52.705) (size 1.5) (drill 0.7) (layers F.Cu B.Cu) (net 5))
 (segment (start 86.36 52.705) (end 99.06 52.705) (width 0.25) (layer F.Cu) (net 5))
 (segment (start 99.06 58.42) (end 99.06 52.705) (width 1) (layer B.Cu) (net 5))
 (via (at 99.06 52.705) (size 1.5) (drill 0.7) (layers F.Cu B.Cu) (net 5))
 (segment (start 86.36 58.42) (end 86.36 52.705) (width 1) (layer B.Cu) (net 5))
 (via (at 86.36 52.705) (size 1.5) (drill 0.7) (layers F.Cu B.Cu) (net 5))
 (segment (start 124.46 63.5) (end 111.913032 63.5) (width 0.25) (layer F.Cu) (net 5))
 (segment (start 109.22 68.58) (end 119.38 68.58) (width 1) (layer B.Cu) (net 5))
 (segment (start 119.38 68.58) (end 124.46 63.5) (width 1) (layer B.Cu) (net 5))
 (segment (start 111.836514 63.423482) (end 111.836516 63.423484) (width 1) (layer F.Cu) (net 5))
 (segment (start 111.76 63.346968) (end 111.836516 63.423484) (width 1) (layer B.Cu) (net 5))
 (via (at 111.836516 63.423484) (size 1.5) (drill 0.7) (layers F.Cu B.Cu) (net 5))
 (segment (start 111.76 58.42) (end 111.76 63.346968) (width 1) (layer B.Cu) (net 5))
 (segment (start 111.913032 63.5) (end 111.836516 63.423484) (width 1) (layer F.Cu) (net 5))
 (segment (start 124.46 63.5) (end 124.46 58.42) (width 1) (layer B.Cu) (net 5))
 (via (at 124.46 63.5) (size 1.5) (layers F.Cu B.Cu) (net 5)))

